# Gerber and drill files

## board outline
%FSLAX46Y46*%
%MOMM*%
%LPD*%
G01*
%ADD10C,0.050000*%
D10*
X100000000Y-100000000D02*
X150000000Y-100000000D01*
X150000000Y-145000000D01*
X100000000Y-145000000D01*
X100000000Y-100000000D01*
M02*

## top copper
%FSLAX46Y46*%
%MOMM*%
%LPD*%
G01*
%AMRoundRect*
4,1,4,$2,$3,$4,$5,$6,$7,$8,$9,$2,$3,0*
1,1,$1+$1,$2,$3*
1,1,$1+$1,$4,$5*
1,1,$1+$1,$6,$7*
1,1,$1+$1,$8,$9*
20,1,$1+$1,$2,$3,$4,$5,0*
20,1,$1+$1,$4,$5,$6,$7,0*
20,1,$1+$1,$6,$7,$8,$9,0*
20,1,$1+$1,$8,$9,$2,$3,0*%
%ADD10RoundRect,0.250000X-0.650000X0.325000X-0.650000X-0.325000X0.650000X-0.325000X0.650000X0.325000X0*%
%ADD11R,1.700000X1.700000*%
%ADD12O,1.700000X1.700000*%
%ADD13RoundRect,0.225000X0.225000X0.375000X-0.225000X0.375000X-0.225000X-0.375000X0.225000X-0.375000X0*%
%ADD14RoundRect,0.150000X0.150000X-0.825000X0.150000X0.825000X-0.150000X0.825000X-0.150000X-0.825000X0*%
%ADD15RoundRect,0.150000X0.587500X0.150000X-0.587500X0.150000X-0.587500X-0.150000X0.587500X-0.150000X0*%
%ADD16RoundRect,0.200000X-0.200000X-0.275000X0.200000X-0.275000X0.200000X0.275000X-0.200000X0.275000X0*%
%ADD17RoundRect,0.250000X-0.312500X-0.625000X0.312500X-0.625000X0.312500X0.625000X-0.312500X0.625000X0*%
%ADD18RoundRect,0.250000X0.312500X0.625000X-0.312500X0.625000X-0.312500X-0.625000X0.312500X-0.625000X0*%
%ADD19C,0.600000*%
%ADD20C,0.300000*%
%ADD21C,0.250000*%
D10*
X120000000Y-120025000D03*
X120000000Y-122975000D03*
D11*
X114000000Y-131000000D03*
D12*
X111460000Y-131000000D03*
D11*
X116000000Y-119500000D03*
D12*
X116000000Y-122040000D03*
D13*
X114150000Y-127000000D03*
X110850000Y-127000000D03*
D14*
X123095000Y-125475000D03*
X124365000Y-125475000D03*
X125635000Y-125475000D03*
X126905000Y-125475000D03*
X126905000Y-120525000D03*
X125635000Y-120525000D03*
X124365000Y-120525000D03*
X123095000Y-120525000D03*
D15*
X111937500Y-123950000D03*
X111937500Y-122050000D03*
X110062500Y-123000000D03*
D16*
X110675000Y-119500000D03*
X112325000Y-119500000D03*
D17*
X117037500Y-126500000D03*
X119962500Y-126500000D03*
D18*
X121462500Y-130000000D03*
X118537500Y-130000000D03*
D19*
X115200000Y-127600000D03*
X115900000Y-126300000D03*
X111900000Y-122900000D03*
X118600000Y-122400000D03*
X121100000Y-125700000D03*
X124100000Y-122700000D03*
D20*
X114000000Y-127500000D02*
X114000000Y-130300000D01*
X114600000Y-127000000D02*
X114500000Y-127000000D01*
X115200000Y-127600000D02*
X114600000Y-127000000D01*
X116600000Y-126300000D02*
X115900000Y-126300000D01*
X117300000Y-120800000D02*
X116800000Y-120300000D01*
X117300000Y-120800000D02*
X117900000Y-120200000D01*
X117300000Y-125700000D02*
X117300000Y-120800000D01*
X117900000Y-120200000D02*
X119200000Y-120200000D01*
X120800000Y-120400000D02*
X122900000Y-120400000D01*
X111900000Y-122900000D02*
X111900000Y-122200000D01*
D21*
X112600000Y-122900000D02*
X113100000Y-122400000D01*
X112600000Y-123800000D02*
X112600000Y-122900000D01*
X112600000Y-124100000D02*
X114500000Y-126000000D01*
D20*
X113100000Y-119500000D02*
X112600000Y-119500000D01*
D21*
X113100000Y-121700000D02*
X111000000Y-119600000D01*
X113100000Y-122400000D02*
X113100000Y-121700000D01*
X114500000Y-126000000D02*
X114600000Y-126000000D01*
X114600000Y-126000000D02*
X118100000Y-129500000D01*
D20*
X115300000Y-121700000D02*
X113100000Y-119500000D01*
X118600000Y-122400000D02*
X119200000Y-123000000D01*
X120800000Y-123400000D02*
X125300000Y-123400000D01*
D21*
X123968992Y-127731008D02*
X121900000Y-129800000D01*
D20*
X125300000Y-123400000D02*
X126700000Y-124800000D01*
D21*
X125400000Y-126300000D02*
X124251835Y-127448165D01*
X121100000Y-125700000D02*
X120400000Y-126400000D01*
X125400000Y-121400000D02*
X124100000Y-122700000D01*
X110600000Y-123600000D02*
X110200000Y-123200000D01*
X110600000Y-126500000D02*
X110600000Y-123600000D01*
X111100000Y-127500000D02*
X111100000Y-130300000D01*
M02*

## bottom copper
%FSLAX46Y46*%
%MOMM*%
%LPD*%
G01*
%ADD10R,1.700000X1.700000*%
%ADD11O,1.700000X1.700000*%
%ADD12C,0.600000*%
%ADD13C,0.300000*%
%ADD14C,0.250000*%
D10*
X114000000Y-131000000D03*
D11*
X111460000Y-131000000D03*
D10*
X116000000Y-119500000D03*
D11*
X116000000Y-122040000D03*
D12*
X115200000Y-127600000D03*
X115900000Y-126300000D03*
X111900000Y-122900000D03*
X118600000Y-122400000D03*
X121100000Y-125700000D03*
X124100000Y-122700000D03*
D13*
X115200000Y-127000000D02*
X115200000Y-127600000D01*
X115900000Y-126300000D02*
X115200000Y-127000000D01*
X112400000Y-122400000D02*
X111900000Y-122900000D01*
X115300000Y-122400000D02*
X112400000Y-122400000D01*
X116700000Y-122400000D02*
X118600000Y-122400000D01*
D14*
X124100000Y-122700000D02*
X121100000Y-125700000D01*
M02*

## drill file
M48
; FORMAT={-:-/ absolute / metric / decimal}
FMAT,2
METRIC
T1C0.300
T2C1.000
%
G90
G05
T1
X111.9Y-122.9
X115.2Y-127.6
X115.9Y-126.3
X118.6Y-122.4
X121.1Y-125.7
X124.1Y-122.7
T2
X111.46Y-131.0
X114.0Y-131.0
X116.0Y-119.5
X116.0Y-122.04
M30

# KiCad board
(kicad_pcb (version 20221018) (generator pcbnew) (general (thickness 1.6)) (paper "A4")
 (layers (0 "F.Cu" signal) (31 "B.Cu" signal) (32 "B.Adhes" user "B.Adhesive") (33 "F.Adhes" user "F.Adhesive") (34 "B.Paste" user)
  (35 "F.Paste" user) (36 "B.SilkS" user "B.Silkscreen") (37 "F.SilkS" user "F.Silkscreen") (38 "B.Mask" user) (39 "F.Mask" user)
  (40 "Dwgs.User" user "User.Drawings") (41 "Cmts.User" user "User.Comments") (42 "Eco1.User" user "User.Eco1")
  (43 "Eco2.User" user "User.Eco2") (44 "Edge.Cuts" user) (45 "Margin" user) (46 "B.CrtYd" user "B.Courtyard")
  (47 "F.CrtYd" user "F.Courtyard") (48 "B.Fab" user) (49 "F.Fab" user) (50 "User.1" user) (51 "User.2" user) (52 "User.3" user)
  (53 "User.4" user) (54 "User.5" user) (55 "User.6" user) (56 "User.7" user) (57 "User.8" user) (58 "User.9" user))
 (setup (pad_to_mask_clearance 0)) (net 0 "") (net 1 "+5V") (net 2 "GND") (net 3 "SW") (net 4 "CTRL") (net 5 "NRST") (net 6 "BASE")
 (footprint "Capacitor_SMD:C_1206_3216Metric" (layer "F.Cu") (at 120 121.5 -90)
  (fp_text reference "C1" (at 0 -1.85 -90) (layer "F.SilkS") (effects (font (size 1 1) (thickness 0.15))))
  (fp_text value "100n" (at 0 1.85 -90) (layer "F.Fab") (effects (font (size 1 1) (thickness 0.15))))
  (pad "1" smd roundrect (at -1.475 0 270) (size 1.15 1.8) (layers "F.Cu" "F.Paste" "F.Mask") (roundrect_rratio 0.217391) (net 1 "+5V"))
  (pad "2" smd roundrect (at 1.475 0 270) (size 1.15 1.8) (layers "F.Cu" "F.Paste" "F.Mask") (roundrect_rratio 0.217391) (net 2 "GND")))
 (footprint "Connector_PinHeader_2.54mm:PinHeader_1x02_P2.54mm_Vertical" (layer "F.Cu") (at 114 131 -90)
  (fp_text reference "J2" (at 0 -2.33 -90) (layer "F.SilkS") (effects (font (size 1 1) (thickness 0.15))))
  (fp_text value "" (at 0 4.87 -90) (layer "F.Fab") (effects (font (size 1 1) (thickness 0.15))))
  (pad "1" thru_hole rect (at 0 0 270) (size 1.7 1.7) (drill 1) (layers "*.Cu" "*.Mask") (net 1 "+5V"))
  (pad "2" thru_hole oval (at 0 2.54 270) (size 1.7 1.7) (drill 1) (layers "*.Cu" "*.Mask") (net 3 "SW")))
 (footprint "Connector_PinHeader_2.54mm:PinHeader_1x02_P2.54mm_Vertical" (layer "F.Cu") (at 116 119.5)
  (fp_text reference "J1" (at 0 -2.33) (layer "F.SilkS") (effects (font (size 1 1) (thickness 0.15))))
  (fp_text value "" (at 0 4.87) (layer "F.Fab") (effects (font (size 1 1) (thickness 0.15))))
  (pad "1" thru_hole rect (at 0 0) (size 1.7 1.7) (drill 1) (layers "*.Cu" "*.Mask") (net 1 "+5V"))
  (pad "2" thru_hole oval (at 0 2.54) (size 1.7 1.7) (drill 1) (layers "*.Cu" "*.Mask") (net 2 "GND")))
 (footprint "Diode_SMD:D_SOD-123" (layer "F.Cu") (at 112.5 127 180)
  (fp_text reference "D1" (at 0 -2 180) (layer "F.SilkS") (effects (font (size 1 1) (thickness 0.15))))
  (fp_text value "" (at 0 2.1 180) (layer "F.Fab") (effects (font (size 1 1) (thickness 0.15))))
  (pad "1" smd roundrect (at -1.65 0 180) (size 0.9 1.2) (layers "F.Cu" "F.Paste" "F.Mask") (roundrect_rratio 0.25) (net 1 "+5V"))
  (pad "2" smd roundrect (at 1.65 0 180) (size 0.9 1.2) (layers "F.Cu" "F.Paste" "F.Mask") (roundrect_rratio 0.25) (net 3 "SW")))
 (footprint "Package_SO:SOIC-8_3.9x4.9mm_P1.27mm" (layer "F.Cu") (at 125 123 90)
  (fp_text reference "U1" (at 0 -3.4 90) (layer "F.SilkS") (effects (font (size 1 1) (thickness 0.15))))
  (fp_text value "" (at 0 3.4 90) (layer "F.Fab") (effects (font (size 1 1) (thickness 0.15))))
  (pad "1" smd roundrect (at -2.475 -1.905 90) (size 1.95 0.6) (layers "F.Cu" "F.Paste" "F.Mask") (roundrect_rratio 0.25))
  (pad "2" smd roundrect (at -2.475 -0.635 90) (size 1.95 0.6) (layers "F.Cu" "F.Paste" "F.Mask") (roundrect_rratio 0.25))
  (pad "3" smd roundrect (at -2.475 0.635 90) (size 1.95 0.6) (layers "F.Cu" "F.Paste" "F.Mask") (roundrect_rratio 0.25) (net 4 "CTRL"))
  (pad "4" smd roundrect (at -2.475 1.905 90) (size 1.95 0.6) (layers "F.Cu" "F.Paste" "F.Mask") (roundrect_rratio 0.25) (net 2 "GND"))
  (pad "5" smd roundrect (at 2.475 1.905 90) (size 1.95 0.6) (layers "F.Cu" "F.Paste" "F.Mask") (roundrect_rratio 0.25))
  (pad "6" smd roundrect (at 2.475 0.635 90) (size 1.95 0.6) (layers "F.Cu" "F.Paste" "F.Mask") (roundrect_rratio 0.25) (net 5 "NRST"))
  (pad "7" smd roundrect (at 2.475 -0.635 90) (size 1.95 0.6) (layers "F.Cu" "F.Paste" "F.Mask") (roundrect_rratio 0.25))
  (pad "8" smd roundrect (at 2.475 -1.905 90) (size 1.95 0.6) (layers "F.Cu" "F.Paste" "F.Mask") (roundrect_rratio 0.25) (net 1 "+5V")))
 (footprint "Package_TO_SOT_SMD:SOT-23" (layer "F.Cu") (at 111 123 180)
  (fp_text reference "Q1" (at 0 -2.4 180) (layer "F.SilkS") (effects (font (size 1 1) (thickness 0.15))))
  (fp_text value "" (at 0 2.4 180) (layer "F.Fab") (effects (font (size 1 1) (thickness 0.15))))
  (pad "1" smd roundrect (at -0.9375 -0.95 180) (size 1.475 0.6) (layers "F.Cu" "F.Paste" "F.Mask") (roundrect_rratio 0.25) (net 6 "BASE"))
  (pad "2" smd roundrect (at -0.9375 0.95 180) (size 1.475 0.6) (layers "F.Cu" "F.Paste" "F.Mask") (roundrect_rratio 0.25) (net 2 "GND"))
  (pad "3" smd roundrect (at 0.9375 0 180) (size 1.475 0.6) (layers "F.Cu" "F.Paste" "F.Mask") (roundrect_rratio 0.25) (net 3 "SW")))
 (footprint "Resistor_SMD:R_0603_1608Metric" (layer "F.Cu") (at 111.5 119.5)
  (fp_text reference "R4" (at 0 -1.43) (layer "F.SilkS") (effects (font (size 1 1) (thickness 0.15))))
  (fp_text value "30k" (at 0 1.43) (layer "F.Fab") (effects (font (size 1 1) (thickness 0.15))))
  (pad "1" smd roundrect (at -0.825 0) (size 0.8 0.95) (layers "F.Cu" "F.Paste" "F.Mask") (roundrect_rratio 0.25) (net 6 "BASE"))
  (pad "2" smd roundrect (at 0.825 0) (size 0.8 0.95) (layers "F.Cu" "F.Paste" "F.Mask") (roundrect_rratio 0.25) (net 2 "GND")))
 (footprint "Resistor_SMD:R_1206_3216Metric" (layer "F.Cu") (at 118.5 126.5)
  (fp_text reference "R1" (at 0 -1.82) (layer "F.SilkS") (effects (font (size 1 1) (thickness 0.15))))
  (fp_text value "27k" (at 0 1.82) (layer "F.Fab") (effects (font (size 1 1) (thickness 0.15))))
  (pad "1" smd roundrect (at -1.4625 0) (size 1.125 1.75) (layers "F.Cu" "F.Paste" "F.Mask") (roundrect_rratio 0.222222) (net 1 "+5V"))
  (pad "2" smd roundrect (at 1.4625 0) (size 1.125 1.75) (layers "F.Cu" "F.Paste" "F.Mask") (roundrect_rratio 0.222222) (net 5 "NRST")))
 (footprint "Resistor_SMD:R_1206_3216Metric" (layer "F.Cu") (at 120 130 180)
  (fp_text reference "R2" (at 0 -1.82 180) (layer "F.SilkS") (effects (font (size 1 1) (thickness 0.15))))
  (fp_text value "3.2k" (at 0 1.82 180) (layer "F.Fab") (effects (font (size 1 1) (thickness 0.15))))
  (pad "1" smd roundrect (at -1.4625 0 180) (size 1.125 1.75) (layers "F.Cu" "F.Paste" "F.Mask") (roundrect_rratio 0.222222) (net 4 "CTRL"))
  (pad "2" smd roundrect (at 1.4625 0 180) (size 1.125 1.75) (layers "F.Cu" "F.Paste" "F.Mask") (roundrect_rratio 0.222222) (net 6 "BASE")))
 (gr_rect (start 100 100) (end 150 145) (stroke (width 0.05) (type default)) (fill none) (layer "Edge.Cuts"))
 (segment (start 114 127.5) (end 114 130.3) (width 0.3) (layer "F.Cu") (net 1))
 (segment (start 114.6 127) (end 114.5 127) (width 0.3) (layer "F.Cu") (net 1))
 (segment (start 115.2 127.6) (end 114.6 127) (width 0.3) (layer "F.Cu") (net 1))
 (segment (start 116.6 126.3) (end 115.9 126.3) (width 0.3) (layer "F.Cu") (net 1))
 (segment (start 117.3 120.8) (end 116.8 120.3) (width 0.3) (layer "F.Cu") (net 1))
 (segment (start 117.3 120.8) (end 117.9 120.2) (width 0.3) (layer "F.Cu") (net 1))
 (segment (start 117.3 125.7) (end 117.3 120.8) (width 0.3) (layer "F.Cu") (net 1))
 (segment (start 117.9 120.2) (end 119.2 120.2) (width 0.3) (layer "F.Cu") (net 1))
 (segment (start 120.8 120.4) (end 122.9 120.4) (width 0.3) (layer "F.Cu") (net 1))
 (via (at 115.2 127.6) (size 0.6) (drill 0.3) (layers "F.Cu" "B.Cu") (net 1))
 (via (at 115.9 126.3) (size 0.6) (drill 0.3) (layers "F.Cu" "B.Cu") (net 1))
 (segment (start 111.9 122.9) (end 111.9 122.2) (width 0.3) (layer "F.Cu") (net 2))
 (segment (start 112.6 122.9) (end 113.1 122.4) (width 0.25) (layer "F.Cu") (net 6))
 (segment (start 112.6 123.8) (end 112.6 122.9) (width 0.25) (layer "F.Cu") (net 6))
 (segment (start 112.6 124.1) (end 114.5 126) (width 0.25) (layer "F.Cu") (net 6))
 (segment (start 113.1 119.5) (end 112.6 119.5) (width 0.3) (layer "F.Cu") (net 2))
 (segment (start 113.1 121.7) (end 111 119.6) (width 0.25) (layer "F.Cu") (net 6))
 (segment (start 113.1 122.4) (end 113.1 121.7) (width 0.25) (layer "F.Cu") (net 6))
 (segment (start 114.5 126) (end 114.6 126) (width 0.25) (layer "F.Cu") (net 6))
 (segment (start 114.6 126) (end 118.1 129.5) (width 0.25) (layer "F.Cu") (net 6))
 (segment (start 115.2 127) (end 115.2 127.6) (width 0.3) (layer "B.Cu") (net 1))
 (segment (start 115.3 121.7) (end 113.1 119.5) (width 0.3) (layer "F.Cu") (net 2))
 (segment (start 115.9 126.3) (end 115.2 127) (width 0.3) (layer "B.Cu") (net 1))
 (segment (start 118.6 122.4) (end 119.2 123) (width 0.3) (layer "F.Cu") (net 2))
 (segment (start 120.8 123.4) (end 125.3 123.4) (width 0.3) (layer "F.Cu") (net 2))
 (segment (start 123.968992 127.731008) (end 121.9 129.8) (width 0.25) (layer "F.Cu") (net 4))
 (segment (start 125.3 123.4) (end 126.7 124.8) (width 0.3) (layer "F.Cu") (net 2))
 (segment (start 125.4 126.3) (end 124.251835 127.448165) (width 0.25) (layer "F.Cu") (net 4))
 (via (at 111.9 122.9) (size 0.6) (drill 0.3) (layers "F.Cu" "B.Cu") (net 2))
 (via (at 118.6 122.4) (size 0.6) (drill 0.3) (layers "F.Cu" "B.Cu") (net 2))
 (segment (start 112.4 122.4) (end 111.9 122.9) (width 0.3) (layer "B.Cu") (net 2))
 (segment (start 115.3 122.4) (end 112.4 122.4) (width 0.3) (layer "B.Cu") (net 2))
 (segment (start 116.7 122.4) (end 118.6 122.4) (width 0.3) (layer "B.Cu") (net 2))
 (segment (start 121.1 125.7) (end 120.4 126.4) (width 0.25) (layer "F.Cu") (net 5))
 (segment (start 125.4 121.4) (end 124.1 122.7) (width 0.25) (layer "F.Cu") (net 5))
 (via (at 121.1 125.7) (size 0.6) (drill 0.3) (layers "F.Cu" "B.Cu") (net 5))
 (via (at 124.1 122.7) (size 0.6) (drill 0.3) (layers "F.Cu" "B.Cu") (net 5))
 (segment (start 110.6 123.6) (end 110.2 123.2) (width 0.25) (layer "F.Cu") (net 3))
 (segment (start 110.6 126.5) (end 110.6 123.6) (width 0.25) (layer "F.Cu") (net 3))
 (segment (start 111.1 127.5) (end 111.1 130.3) (width 0.25) (layer "F.Cu") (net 3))
 (segment (start 124.1 122.7) (end 121.1 125.7) (width 0.25) (layer "B.Cu") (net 5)))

